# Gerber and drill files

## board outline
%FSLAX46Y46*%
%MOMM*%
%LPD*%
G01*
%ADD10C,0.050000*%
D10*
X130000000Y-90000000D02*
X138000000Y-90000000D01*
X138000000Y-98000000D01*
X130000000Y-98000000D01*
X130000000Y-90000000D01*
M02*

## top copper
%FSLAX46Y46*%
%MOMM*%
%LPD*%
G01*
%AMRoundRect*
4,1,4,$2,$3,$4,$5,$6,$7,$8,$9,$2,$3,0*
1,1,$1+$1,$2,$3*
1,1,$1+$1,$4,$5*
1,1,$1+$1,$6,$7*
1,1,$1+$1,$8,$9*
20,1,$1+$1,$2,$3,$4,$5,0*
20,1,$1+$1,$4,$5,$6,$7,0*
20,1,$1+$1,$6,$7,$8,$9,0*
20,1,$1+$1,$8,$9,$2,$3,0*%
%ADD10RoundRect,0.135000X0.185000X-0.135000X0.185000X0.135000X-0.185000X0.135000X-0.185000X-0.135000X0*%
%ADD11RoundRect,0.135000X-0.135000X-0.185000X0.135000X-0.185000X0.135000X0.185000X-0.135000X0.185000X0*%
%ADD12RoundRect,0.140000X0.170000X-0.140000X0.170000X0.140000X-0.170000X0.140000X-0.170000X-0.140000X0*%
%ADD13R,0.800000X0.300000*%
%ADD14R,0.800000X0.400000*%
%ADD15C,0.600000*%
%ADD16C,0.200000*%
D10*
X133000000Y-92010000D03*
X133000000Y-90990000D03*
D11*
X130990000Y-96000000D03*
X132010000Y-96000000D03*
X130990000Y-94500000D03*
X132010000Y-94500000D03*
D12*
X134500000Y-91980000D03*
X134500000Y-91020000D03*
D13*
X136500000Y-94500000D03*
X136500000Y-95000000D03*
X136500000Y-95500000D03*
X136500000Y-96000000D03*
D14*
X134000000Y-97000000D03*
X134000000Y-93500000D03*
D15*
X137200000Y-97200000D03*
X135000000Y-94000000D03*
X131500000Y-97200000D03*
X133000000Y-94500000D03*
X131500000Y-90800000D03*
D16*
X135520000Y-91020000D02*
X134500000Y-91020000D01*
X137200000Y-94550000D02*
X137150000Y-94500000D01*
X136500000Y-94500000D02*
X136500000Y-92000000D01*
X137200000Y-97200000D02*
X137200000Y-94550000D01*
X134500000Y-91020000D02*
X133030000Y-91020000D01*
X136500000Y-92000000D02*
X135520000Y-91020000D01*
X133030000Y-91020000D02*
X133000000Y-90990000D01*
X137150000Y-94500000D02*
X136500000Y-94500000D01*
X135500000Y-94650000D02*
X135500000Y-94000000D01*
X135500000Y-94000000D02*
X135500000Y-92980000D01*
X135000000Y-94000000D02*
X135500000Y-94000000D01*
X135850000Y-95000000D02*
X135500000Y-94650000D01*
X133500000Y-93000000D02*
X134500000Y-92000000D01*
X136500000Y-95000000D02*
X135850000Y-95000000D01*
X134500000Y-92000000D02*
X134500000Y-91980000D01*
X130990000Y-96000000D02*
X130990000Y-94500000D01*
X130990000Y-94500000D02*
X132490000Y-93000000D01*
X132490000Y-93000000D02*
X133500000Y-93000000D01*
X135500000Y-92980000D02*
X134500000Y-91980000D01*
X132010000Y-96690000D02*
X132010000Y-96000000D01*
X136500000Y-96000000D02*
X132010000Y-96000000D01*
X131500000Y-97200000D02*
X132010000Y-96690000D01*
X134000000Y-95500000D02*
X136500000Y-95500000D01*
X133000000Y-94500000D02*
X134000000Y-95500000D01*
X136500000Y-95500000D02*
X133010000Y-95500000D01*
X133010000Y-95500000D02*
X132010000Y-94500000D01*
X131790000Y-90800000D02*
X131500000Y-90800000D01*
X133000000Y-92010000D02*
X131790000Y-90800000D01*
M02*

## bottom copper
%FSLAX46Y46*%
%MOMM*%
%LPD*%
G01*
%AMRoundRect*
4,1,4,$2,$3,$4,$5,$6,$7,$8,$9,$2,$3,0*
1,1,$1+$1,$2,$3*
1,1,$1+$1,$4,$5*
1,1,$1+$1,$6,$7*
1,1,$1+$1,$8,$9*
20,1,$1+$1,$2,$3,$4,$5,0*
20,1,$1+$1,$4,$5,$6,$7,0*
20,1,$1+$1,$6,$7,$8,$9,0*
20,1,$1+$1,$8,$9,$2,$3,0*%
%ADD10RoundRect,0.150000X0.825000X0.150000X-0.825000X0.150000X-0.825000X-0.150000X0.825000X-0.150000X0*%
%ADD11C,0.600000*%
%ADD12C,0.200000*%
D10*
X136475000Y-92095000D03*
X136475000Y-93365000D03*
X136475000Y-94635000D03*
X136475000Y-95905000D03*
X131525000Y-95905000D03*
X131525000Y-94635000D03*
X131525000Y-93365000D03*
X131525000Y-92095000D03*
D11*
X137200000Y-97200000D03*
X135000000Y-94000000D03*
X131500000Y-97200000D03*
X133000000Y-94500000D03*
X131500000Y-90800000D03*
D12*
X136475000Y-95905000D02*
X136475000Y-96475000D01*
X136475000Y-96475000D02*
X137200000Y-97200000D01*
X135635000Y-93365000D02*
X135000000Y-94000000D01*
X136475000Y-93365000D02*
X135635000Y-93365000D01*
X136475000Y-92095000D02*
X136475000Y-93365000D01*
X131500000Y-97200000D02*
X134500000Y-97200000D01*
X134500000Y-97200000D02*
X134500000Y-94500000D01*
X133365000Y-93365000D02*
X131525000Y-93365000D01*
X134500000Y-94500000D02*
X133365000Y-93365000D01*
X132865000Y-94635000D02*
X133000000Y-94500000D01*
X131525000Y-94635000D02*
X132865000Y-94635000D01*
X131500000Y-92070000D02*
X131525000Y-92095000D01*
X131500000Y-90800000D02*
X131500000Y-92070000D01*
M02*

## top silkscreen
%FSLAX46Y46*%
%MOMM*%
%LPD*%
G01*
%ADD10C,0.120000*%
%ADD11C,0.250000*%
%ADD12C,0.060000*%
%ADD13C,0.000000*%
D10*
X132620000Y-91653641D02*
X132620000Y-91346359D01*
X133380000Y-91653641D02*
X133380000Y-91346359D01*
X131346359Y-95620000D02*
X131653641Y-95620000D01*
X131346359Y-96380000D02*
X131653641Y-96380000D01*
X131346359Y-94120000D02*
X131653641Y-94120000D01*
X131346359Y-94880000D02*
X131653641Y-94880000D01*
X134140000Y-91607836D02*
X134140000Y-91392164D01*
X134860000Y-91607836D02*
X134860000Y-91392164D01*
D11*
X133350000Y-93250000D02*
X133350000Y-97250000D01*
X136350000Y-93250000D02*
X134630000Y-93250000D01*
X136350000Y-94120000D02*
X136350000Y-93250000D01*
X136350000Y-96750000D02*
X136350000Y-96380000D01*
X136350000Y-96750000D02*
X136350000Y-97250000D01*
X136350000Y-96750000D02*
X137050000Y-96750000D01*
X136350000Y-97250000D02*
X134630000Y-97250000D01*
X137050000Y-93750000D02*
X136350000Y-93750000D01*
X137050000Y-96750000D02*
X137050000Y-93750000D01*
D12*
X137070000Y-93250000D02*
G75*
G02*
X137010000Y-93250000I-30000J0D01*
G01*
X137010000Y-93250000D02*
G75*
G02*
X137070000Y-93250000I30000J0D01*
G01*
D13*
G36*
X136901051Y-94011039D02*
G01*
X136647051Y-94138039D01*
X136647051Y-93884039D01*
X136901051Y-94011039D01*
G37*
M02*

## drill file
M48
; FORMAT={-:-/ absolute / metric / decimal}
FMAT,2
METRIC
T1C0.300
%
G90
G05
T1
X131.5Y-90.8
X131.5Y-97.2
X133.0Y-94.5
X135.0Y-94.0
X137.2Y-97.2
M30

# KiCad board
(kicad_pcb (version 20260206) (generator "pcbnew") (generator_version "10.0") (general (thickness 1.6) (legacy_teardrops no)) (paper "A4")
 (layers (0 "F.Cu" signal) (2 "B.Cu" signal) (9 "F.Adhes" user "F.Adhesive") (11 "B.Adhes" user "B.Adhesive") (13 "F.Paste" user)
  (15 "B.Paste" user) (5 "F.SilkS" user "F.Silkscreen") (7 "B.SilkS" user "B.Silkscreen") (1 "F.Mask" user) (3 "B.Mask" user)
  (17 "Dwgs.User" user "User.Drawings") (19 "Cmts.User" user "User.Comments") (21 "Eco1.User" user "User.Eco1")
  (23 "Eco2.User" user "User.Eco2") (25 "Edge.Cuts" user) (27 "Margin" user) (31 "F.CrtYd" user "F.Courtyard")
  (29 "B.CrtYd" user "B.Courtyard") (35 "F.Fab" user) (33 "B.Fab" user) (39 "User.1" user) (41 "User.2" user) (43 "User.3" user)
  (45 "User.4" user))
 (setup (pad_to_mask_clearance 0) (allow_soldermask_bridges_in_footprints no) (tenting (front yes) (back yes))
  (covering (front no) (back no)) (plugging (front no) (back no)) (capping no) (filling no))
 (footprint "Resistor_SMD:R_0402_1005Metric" (layer "F.Cu") (at 133 91.5 90)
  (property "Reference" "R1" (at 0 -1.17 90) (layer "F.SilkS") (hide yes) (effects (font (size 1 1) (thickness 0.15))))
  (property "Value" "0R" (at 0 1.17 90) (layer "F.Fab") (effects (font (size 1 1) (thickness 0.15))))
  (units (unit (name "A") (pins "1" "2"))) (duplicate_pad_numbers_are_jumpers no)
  (fp_line (start -0.153641 -0.38) (end 0.153641 -0.38) (stroke (width 0.12) (type solid)) (layer "F.SilkS"))
  (fp_line (start -0.153641 0.38) (end 0.153641 0.38) (stroke (width 0.12) (type solid)) (layer "F.SilkS"))
  (pad "1" smd roundrect (at -0.51 0 90) (size 0.54 0.64) (layers "F.Cu" "F.Mask" "F.Paste") (roundrect_rratio 0.25) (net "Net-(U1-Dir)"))
  (pad "2" smd roundrect (at 0.51 0 90) (size 0.54 0.64) (layers "F.Cu" "F.Mask" "F.Paste") (roundrect_rratio 0.25) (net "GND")))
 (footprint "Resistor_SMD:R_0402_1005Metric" (layer "F.Cu") (at 131.5 96)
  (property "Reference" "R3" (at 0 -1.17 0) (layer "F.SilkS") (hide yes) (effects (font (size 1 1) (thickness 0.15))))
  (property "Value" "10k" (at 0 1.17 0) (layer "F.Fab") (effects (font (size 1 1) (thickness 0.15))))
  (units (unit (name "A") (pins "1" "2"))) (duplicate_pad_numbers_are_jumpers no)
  (fp_line (start -0.153641 -0.38) (end 0.153641 -0.38) (stroke (width 0.12) (type solid)) (layer "F.SilkS"))
  (fp_line (start -0.153641 0.38) (end 0.153641 0.38) (stroke (width 0.12) (type solid)) (layer "F.SilkS"))
  (pad "1" smd roundrect (at -0.51 0) (size 0.54 0.64) (layers "F.Cu" "F.Mask" "F.Paste") (roundrect_rratio 0.25) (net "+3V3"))
  (pad "2" smd roundrect (at 0.51 0) (size 0.54 0.64) (layers "F.Cu" "F.Mask" "F.Paste") (roundrect_rratio 0.25) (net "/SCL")))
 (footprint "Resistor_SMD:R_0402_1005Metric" (layer "F.Cu") (at 131.5 94.5)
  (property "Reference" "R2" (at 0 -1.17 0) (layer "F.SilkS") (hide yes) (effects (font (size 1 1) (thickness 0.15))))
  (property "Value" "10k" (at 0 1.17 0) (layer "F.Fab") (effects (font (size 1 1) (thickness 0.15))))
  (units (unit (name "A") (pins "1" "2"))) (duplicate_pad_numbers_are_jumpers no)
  (fp_line (start -0.153641 -0.38) (end 0.153641 -0.38) (stroke (width 0.12) (type solid)) (layer "F.SilkS"))
  (fp_line (start -0.153641 0.38) (end 0.153641 0.38) (stroke (width 0.12) (type solid)) (layer "F.SilkS"))
  (pad "1" smd roundrect (at -0.51 0) (size 0.54 0.64) (layers "F.Cu" "F.Mask" "F.Paste") (roundrect_rratio 0.25) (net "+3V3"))
  (pad "2" smd roundrect (at 0.51 0) (size 0.54 0.64) (layers "F.Cu" "F.Mask" "F.Paste") (roundrect_rratio 0.25) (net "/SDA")))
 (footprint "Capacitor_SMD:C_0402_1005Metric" (layer "F.Cu") (at 134.5 91.5 90)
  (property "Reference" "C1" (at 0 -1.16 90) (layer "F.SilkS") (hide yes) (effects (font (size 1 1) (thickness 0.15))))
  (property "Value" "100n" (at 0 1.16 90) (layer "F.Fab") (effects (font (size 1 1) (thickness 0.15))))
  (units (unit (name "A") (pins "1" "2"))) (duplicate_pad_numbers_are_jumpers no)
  (fp_line (start -0.107836 -0.36) (end 0.107836 -0.36) (stroke (width 0.12) (type solid)) (layer "F.SilkS"))
  (fp_line (start -0.107836 0.36) (end 0.107836 0.36) (stroke (width 0.12) (type solid)) (layer "F.SilkS"))
  (pad "1" smd roundrect (at -0.48 0 90) (size 0.56 0.62) (layers "F.Cu" "F.Mask" "F.Paste") (roundrect_rratio 0.25) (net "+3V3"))
  (pad "2" smd roundrect (at 0.48 0 90) (size 0.56 0.62) (layers "F.Cu" "F.Mask" "F.Paste") (roundrect_rratio 0.25) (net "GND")))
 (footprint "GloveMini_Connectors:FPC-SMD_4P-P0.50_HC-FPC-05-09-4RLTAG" (layer "F.Cu") (at 135.25 95.25 90)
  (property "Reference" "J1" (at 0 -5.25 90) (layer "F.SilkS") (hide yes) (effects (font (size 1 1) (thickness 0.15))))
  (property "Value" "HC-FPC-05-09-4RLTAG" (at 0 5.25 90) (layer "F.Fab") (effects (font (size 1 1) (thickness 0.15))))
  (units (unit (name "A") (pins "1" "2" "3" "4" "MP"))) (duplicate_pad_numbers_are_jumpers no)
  (fp_line (start 2 -1.9) (end -2 -1.9) (stroke (width 0.25) (type solid)) (layer "F.SilkS"))
  (fp_line (start 2 1.1) (end 2 -0.62) (stroke (width 0.25) (type solid)) (layer "F.SilkS"))
  (fp_line (start 1.13 1.1) (end 2 1.1) (stroke (width 0.25) (type solid)) (layer "F.SilkS"))
  (fp_line (start -1.5 1.1) (end -1.13 1.1) (stroke (width 0.25) (type solid)) (layer "F.SilkS"))
  (fp_line (start -1.5 1.1) (end -2 1.1) (stroke (width 0.25) (type solid)) (layer "F.SilkS"))
  (fp_line (start -1.5 1.1) (end -1.5 1.8) (stroke (width 0.25) (type solid)) (layer "F.SilkS"))
  (fp_line (start -2 1.1) (end -2 -0.62) (stroke (width 0.25) (type solid)) (layer "F.SilkS"))
  (fp_line (start 1.5 1.8) (end 1.5 1.1) (stroke (width 0.25) (type solid)) (layer "F.SilkS"))
  (fp_line (start -1.5 1.8) (end 1.5 1.8) (stroke (width 0.25) (type solid)) (layer "F.SilkS"))
  (fp_circle (center 2 1.79) (end 2.03 1.79) (stroke (width 0.06) (type solid)) (fill no) (layer "F.SilkS"))
  (fp_poly
   (pts (xy 1.238961 1.651051) (xy 1.365961 1.397051) (xy 1.238961 1.524051) (xy 1.365961 1.397051) (xy 1.111961 1.397051)
    (xy 1.238961 1.651051))
   (stroke (width 0) (type solid)) (fill yes) (layer "F.SilkS"))
  (pad "1" smd rect (at 0.75 1.25 270) (size 0.3 0.8) (layers "F.Cu" "F.Mask" "F.Paste") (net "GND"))
  (pad "2" smd rect (at 0.25 1.25 270) (size 0.3 0.8) (layers "F.Cu" "F.Mask" "F.Paste") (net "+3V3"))
  (pad "3" smd rect (at -0.25 1.25 270) (size 0.3 0.8) (layers "F.Cu" "F.Mask" "F.Paste") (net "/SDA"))
  (pad "4" smd rect (at -0.75 1.25 270) (size 0.3 0.8) (layers "F.Cu" "F.Mask" "F.Paste") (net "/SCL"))
  (pad "MP" smd rect (at -1.75 -1.25 270) (size 0.4 0.8) (layers "F.Cu" "F.Mask" "F.Paste") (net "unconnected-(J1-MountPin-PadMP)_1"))
  (pad "MP" smd rect (at 1.75 -1.25 270) (size 0.4 0.8) (layers "F.Cu" "F.Mask" "F.Paste") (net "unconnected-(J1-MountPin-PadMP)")))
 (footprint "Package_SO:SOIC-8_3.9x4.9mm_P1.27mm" (layer "B.Cu") (at 134 94 180)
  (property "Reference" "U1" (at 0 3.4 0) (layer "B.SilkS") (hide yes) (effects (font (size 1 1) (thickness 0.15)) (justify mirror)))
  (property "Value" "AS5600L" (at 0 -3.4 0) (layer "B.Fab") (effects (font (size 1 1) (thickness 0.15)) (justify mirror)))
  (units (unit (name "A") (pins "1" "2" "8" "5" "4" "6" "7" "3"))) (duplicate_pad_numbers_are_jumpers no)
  (pad "1" smd roundrect (at -2.475 1.905 180) (size 1.95 0.6) (layers "B.Cu" "B.Mask" "B.Paste") (roundrect_rratio 0.25) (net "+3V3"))
  (pad "2" smd roundrect (at -2.475 0.635 180) (size 1.95 0.6) (layers "B.Cu" "B.Mask" "B.Paste") (roundrect_rratio 0.25) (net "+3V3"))
  (pad "3" smd roundrect (at -2.475 -0.635 180) (size 1.95 0.6) (layers "B.Cu" "B.Mask" "B.Paste") (roundrect_rratio 0.25)
   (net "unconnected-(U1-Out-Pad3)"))
  (pad "4" smd roundrect (at -2.475 -1.905 180) (size 1.95 0.6) (layers "B.Cu" "B.Mask" "B.Paste") (roundrect_rratio 0.25) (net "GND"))
  (pad "5" smd roundrect (at 2.475 -1.905 180) (size 1.95 0.6) (layers "B.Cu" "B.Mask" "B.Paste") (roundrect_rratio 0.25)
   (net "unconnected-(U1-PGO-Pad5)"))
  (pad "6" smd roundrect (at 2.475 -0.635 180) (size 1.95 0.6) (layers "B.Cu" "B.Mask" "B.Paste") (roundrect_rratio 0.25) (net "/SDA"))
  (pad "7" smd roundrect (at 2.475 0.635 180) (size 1.95 0.6) (layers "B.Cu" "B.Mask" "B.Paste") (roundrect_rratio 0.25) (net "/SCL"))
  (pad "8" smd roundrect (at 2.475 1.905 180) (size 1.95 0.6) (layers "B.Cu" "B.Mask" "B.Paste") (roundrect_rratio 0.25)
   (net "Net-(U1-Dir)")))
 (gr_rect (start 130 90) (end 138 98) (stroke (width 0.05) (type solid)) (fill no) (layer "Edge.Cuts"))
 (segment (start 135.52 91.02) (end 134.5 91.02) (width 0.2) (layer "F.Cu") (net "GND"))
 (segment (start 137.2 94.55) (end 137.15 94.5) (width 0.2) (layer "F.Cu") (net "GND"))
 (segment (start 136.5 94.5) (end 136.5 92) (width 0.2) (layer "F.Cu") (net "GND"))
 (segment (start 137.2 97.2) (end 137.2 94.55) (width 0.2) (layer "F.Cu") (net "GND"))
 (segment (start 134.5 91.02) (end 133.03 91.02) (width 0.2) (layer "F.Cu") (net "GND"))
 (segment (start 136.5 92) (end 135.52 91.02) (width 0.2) (layer "F.Cu") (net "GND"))
 (segment (start 133.03 91.02) (end 133 90.99) (width 0.2) (layer "F.Cu") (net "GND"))
 (segment (start 137.15 94.5) (end 136.5 94.5) (width 0.2) (layer "F.Cu") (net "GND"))
 (via (at 137.2 97.2) (size 0.6) (drill 0.3) (layers "F.Cu" "B.Cu") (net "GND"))
 (segment (start 136.475 95.905) (end 136.475 96.475) (width 0.2) (layer "B.Cu") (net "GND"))
 (segment (start 136.475 96.475) (end 137.2 97.2) (width 0.2) (layer "B.Cu") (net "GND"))
 (segment (start 135.5 94.65) (end 135.5 94) (width 0.2) (layer "F.Cu") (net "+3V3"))
 (segment (start 135.5 94) (end 135.5 92.98) (width 0.2) (layer "F.Cu") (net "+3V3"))
 (segment (start 135 94) (end 135.5 94) (width 0.2) (layer "F.Cu") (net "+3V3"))
 (segment (start 135.85 95) (end 135.5 94.65) (width 0.2) (layer "F.Cu") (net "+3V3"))
 (segment (start 133.5 93) (end 134.5 92) (width 0.2) (layer "F.Cu") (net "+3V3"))
 (segment (start 136.5 95) (end 135.85 95) (width 0.2) (layer "F.Cu") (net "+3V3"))
 (segment (start 134.5 92) (end 134.5 91.98) (width 0.2) (layer "F.Cu") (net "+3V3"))
 (segment (start 130.99 96) (end 130.99 94.5) (width 0.2) (layer "F.Cu") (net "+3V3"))
 (segment (start 130.99 94.5) (end 132.49 93) (width 0.2) (layer "F.Cu") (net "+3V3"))
 (segment (start 132.49 93) (end 133.5 93) (width 0.2) (layer "F.Cu") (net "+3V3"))
 (segment (start 135.5 92.98) (end 134.5 91.98) (width 0.2) (layer "F.Cu") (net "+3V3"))
 (via (at 135 94) (size 0.6) (drill 0.3) (layers "F.Cu" "B.Cu") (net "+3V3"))
 (segment (start 135.635 93.365) (end 135 94) (width 0.2) (layer "B.Cu") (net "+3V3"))
 (segment (start 136.475 93.365) (end 135.635 93.365) (width 0.2) (layer "B.Cu") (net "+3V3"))
 (segment (start 136.475 92.095) (end 136.475 93.365) (width 0.2) (layer "B.Cu") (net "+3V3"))
 (segment (start 132.01 96.69) (end 132.01 96) (width 0.2) (layer "F.Cu") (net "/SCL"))
 (segment (start 136.5 96) (end 132.01 96) (width 0.2) (layer "F.Cu") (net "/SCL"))
 (segment (start 131.5 97.2) (end 132.01 96.69) (width 0.2) (layer "F.Cu") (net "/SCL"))
 (via (at 131.5 97.2) (size 0.6) (drill 0.3) (layers "F.Cu" "B.Cu") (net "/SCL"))
 (segment (start 131.5 97.2) (end 134.5 97.2) (width 0.2) (layer "B.Cu") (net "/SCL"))
 (segment (start 134.5 97.2) (end 134.5 94.5) (width 0.2) (layer "B.Cu") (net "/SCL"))
 (segment (start 133.365 93.365) (end 131.525 93.365) (width 0.2) (layer "B.Cu") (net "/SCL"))
 (segment (start 134.5 94.5) (end 133.365 93.365) (width 0.2) (layer "B.Cu") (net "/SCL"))
 (segment (start 134 95.5) (end 136.5 95.5) (width 0.2) (layer "F.Cu") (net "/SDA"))
 (segment (start 133 94.5) (end 134 95.5) (width 0.2) (layer "F.Cu") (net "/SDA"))
 (segment (start 136.5 95.5) (end 133.01 95.5) (width 0.2) (layer "F.Cu") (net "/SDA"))
 (segment (start 133.01 95.5) (end 132.01 94.5) (width 0.2) (layer "F.Cu") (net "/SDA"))
 (via (at 133 94.5) (size 0.6) (drill 0.3) (layers "F.Cu" "B.Cu") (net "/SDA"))
 (segment (start 132.865 94.635) (end 133 94.5) (width 0.2) (layer "B.Cu") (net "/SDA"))
 (segment (start 131.525 94.635) (end 132.865 94.635) (width 0.2) (layer "B.Cu") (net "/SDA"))
 (segment (start 131.79 90.8) (end 131.5 90.8) (width 0.2) (layer "F.Cu") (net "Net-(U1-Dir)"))
 (segment (start 133 92.01) (end 131.79 90.8) (width 0.2) (layer "F.Cu") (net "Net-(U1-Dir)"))
 (via (at 131.5 90.8) (size 0.6) (drill 0.3) (layers "F.Cu" "B.Cu") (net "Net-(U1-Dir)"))
 (segment (start 131.5 92.07) (end 131.525 92.095) (width 0.2) (layer "B.Cu") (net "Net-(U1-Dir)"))
 (segment (start 131.5 90.8) (end 131.5 92.07) (width 0.2) (layer "B.Cu") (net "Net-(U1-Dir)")))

